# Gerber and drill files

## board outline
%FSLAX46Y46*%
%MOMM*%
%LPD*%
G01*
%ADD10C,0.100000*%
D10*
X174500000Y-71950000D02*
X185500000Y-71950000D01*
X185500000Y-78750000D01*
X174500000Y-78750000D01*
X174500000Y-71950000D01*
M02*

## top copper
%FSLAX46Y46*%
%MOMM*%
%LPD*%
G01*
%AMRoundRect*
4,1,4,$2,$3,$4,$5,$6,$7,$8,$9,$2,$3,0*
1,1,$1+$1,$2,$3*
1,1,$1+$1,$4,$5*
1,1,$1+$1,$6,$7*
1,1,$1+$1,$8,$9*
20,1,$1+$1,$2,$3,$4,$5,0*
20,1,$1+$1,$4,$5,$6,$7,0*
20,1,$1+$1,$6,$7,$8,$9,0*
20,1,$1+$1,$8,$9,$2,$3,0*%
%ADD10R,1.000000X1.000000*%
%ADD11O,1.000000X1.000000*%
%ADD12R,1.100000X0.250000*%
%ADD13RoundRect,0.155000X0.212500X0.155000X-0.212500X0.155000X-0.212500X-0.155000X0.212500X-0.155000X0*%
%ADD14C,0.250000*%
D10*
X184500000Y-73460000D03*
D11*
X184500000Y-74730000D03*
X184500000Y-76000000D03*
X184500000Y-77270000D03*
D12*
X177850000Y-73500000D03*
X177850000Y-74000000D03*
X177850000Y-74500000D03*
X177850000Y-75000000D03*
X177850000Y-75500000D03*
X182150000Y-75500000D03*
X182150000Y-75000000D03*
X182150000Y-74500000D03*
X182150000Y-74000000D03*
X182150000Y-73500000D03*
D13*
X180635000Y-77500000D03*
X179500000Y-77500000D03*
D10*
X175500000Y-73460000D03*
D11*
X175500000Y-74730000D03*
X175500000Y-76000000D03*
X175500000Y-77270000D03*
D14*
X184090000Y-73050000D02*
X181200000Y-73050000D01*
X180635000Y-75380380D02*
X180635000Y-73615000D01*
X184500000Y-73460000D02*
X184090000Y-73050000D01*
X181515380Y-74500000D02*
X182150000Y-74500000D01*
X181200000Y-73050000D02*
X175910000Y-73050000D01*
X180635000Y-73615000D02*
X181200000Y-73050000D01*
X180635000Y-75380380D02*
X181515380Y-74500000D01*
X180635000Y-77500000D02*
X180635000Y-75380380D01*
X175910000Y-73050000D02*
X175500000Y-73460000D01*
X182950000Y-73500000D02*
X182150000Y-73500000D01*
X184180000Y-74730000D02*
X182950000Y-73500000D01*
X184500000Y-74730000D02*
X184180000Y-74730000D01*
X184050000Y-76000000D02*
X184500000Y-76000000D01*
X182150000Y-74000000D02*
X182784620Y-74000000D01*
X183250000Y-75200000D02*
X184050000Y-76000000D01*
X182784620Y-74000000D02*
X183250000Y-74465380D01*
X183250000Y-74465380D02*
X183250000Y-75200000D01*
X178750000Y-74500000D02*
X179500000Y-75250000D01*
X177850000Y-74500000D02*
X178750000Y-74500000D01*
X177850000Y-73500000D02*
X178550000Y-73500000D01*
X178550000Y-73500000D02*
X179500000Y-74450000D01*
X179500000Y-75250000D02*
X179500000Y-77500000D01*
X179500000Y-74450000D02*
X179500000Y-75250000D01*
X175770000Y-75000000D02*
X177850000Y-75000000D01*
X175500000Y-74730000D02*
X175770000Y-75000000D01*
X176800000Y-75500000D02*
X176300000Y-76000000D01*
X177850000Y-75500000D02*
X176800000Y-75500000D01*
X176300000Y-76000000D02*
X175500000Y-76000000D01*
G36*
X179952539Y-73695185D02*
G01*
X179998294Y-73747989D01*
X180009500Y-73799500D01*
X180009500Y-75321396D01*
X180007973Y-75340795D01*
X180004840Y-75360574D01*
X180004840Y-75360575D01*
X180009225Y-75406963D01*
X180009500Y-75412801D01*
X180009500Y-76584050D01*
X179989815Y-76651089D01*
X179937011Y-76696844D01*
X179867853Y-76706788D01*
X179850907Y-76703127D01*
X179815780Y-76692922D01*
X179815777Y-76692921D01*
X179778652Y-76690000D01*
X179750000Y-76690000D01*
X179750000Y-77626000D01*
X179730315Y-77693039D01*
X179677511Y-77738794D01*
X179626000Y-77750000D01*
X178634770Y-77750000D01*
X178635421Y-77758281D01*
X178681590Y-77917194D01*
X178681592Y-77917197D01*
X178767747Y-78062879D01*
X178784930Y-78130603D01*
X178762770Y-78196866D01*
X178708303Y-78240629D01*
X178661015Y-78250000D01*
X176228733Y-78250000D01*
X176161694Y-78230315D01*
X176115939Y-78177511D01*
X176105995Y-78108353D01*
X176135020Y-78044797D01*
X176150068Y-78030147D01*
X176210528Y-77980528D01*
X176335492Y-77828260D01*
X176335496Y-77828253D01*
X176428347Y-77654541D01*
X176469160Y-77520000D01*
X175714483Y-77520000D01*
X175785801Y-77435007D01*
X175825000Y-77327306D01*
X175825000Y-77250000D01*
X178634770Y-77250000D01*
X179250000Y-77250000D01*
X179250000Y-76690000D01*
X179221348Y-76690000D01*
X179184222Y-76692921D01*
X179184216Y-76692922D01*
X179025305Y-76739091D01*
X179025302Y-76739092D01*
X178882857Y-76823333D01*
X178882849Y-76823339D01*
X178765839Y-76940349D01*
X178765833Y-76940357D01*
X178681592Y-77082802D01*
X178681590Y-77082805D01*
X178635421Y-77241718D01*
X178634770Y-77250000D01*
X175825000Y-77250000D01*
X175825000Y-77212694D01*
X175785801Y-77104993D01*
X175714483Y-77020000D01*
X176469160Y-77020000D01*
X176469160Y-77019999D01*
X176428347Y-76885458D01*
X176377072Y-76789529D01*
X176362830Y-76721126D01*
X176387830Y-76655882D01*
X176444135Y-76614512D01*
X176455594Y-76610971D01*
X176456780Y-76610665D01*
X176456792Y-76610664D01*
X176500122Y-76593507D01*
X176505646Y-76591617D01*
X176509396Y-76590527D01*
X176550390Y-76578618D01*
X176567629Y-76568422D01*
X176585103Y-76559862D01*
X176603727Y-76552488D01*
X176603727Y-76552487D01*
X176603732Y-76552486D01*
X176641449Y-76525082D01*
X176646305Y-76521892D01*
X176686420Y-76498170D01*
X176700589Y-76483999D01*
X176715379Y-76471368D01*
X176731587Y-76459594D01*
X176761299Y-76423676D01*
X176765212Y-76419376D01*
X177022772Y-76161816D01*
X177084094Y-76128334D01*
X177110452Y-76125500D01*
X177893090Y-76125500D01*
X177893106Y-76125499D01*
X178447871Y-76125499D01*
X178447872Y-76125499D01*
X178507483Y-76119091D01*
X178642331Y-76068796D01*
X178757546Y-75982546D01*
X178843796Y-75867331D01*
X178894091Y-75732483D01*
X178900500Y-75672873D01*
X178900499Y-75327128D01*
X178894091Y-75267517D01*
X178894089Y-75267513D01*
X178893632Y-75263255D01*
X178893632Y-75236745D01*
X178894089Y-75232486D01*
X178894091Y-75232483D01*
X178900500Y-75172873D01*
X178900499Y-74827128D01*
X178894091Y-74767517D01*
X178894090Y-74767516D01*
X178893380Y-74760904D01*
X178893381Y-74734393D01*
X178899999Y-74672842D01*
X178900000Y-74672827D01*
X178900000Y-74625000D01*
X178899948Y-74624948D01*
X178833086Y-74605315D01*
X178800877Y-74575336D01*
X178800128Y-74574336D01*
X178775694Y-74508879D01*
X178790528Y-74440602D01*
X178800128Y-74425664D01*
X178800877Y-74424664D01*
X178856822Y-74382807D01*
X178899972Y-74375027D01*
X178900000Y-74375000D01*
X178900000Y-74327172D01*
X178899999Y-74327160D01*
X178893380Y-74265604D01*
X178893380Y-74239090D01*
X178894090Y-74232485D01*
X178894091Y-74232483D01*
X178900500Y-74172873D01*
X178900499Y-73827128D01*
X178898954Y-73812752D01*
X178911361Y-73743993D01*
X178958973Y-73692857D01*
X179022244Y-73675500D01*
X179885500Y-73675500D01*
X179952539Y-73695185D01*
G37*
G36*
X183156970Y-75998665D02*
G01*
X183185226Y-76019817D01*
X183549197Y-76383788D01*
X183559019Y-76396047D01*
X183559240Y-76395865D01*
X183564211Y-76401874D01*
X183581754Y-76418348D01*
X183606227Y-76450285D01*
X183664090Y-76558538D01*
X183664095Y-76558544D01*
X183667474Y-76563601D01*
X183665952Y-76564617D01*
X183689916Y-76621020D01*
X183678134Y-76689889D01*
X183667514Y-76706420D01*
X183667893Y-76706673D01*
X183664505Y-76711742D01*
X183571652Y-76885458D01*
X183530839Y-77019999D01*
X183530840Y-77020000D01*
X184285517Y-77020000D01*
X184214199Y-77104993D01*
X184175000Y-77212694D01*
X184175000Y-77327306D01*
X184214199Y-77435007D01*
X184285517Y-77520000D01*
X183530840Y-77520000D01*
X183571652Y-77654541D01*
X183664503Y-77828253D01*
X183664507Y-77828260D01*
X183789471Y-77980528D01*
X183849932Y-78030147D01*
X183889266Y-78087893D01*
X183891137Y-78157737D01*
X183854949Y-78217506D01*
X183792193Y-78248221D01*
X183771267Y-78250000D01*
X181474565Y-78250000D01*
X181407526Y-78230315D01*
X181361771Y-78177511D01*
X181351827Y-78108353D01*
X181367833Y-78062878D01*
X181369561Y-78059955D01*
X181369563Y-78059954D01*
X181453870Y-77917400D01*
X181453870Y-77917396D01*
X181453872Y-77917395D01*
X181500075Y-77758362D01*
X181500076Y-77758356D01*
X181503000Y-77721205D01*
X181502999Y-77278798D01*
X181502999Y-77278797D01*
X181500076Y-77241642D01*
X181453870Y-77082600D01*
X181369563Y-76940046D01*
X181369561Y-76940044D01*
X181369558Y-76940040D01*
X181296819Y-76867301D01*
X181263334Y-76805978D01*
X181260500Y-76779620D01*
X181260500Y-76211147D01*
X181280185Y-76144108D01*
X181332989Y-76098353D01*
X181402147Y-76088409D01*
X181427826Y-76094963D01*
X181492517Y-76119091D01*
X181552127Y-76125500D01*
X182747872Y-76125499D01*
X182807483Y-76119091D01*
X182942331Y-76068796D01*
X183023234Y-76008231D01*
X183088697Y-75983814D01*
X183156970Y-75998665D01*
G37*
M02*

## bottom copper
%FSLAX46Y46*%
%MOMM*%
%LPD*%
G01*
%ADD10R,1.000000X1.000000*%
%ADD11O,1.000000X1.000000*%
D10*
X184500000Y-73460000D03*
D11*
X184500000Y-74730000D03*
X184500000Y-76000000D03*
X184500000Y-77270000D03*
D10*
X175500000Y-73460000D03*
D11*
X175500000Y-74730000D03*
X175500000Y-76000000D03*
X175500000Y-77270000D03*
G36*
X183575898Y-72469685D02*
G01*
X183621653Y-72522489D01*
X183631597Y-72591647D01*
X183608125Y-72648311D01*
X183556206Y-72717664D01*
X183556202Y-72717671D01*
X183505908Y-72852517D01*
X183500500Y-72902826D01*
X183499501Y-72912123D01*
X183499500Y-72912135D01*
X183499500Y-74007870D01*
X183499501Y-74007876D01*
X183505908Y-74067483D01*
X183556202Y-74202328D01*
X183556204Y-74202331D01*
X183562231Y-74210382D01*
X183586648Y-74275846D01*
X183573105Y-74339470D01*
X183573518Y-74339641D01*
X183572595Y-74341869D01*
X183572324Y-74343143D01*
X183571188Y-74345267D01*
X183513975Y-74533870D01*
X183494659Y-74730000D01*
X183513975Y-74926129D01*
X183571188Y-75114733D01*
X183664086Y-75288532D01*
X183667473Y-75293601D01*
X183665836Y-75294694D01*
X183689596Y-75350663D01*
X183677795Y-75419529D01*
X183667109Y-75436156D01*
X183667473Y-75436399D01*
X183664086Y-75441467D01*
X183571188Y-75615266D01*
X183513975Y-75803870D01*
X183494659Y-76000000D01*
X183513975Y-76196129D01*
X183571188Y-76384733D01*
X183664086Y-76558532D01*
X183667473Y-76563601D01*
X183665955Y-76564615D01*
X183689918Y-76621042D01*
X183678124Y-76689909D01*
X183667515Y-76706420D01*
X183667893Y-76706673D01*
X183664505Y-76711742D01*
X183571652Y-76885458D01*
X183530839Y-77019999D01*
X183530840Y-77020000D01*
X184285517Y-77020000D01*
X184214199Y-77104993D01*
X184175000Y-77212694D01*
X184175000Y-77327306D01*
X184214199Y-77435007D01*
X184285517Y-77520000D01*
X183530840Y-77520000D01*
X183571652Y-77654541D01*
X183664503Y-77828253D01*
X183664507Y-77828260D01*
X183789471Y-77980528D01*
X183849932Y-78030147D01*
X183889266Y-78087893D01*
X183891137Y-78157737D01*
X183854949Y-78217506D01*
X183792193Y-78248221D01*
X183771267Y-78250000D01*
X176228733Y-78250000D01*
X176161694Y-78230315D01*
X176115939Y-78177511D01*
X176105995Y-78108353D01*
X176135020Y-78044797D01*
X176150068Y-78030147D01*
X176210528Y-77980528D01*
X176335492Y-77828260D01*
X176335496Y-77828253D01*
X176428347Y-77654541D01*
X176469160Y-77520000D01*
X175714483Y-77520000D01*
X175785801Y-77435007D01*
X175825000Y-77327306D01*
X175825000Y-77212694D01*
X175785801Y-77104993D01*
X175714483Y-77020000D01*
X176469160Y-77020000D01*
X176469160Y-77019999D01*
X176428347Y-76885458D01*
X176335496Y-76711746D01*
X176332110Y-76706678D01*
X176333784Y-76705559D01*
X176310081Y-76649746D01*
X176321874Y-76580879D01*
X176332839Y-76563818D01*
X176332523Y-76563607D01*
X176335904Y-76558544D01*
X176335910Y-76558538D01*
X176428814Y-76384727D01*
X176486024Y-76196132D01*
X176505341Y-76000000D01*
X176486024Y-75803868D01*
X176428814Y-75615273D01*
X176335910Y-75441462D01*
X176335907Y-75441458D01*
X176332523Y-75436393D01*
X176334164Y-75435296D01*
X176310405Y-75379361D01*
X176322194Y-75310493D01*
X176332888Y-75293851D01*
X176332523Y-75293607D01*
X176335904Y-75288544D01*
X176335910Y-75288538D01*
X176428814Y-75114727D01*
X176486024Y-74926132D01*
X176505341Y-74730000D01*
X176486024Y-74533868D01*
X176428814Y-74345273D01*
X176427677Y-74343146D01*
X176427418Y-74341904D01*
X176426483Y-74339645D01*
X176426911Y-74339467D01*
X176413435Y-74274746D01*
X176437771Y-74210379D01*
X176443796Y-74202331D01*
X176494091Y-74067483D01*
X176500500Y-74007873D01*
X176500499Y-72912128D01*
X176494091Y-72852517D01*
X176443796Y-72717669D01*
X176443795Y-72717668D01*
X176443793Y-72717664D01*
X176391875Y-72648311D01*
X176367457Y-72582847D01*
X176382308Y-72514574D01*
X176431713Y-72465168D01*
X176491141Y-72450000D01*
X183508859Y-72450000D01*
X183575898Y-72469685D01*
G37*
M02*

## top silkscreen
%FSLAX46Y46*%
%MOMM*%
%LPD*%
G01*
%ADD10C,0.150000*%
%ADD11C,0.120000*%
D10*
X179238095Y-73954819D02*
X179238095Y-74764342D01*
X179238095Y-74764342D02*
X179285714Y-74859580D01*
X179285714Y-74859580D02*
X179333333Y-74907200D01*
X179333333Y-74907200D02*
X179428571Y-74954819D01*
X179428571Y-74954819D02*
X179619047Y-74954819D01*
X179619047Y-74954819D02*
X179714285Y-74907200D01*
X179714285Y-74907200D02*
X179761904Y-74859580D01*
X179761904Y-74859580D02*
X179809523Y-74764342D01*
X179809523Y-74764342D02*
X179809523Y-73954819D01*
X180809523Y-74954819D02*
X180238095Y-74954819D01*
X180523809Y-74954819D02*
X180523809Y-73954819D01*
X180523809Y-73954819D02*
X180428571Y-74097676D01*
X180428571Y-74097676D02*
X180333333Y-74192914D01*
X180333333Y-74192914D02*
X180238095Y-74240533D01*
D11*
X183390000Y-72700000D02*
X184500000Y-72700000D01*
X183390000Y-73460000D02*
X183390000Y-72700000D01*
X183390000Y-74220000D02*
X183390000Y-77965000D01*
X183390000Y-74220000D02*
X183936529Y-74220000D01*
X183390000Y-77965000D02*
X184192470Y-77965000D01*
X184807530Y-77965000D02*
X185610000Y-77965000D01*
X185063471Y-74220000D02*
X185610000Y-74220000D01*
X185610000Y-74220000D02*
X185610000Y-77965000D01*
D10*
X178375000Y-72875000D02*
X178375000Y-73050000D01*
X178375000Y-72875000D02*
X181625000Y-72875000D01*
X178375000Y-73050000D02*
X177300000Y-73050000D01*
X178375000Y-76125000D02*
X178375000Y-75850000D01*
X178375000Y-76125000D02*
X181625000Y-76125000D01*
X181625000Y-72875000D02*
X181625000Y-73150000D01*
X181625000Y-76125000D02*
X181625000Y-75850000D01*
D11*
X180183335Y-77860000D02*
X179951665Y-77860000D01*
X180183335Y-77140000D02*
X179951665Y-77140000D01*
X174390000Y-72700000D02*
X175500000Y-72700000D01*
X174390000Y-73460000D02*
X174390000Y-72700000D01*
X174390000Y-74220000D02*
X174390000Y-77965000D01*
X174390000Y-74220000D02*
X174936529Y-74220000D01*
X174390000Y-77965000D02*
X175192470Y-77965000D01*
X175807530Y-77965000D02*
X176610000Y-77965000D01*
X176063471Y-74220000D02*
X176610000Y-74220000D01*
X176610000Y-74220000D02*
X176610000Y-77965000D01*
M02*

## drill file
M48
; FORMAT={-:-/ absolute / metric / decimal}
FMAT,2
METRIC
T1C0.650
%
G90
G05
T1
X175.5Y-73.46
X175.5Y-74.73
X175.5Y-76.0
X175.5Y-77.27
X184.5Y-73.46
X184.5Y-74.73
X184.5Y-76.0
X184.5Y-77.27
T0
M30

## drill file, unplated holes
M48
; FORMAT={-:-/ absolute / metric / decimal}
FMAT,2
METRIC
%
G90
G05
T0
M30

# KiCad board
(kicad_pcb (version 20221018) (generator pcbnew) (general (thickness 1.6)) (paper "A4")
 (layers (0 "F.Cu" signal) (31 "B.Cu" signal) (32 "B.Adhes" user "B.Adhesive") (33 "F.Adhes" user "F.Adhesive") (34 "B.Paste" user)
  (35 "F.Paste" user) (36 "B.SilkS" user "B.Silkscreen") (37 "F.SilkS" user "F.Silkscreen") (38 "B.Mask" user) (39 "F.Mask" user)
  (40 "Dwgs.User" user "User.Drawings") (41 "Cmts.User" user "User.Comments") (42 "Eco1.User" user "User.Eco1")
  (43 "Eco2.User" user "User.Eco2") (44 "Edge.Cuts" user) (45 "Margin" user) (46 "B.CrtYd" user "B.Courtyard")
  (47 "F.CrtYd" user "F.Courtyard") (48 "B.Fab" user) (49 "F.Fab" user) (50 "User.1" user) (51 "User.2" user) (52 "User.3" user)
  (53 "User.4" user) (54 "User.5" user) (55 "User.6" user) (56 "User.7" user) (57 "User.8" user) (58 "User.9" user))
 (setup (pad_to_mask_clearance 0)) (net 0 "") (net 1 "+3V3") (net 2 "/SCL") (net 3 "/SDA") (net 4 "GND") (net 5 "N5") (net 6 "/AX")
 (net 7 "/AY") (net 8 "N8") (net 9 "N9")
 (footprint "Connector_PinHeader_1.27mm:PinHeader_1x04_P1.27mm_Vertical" (layer "F.Cu") (at 184.5 73.46)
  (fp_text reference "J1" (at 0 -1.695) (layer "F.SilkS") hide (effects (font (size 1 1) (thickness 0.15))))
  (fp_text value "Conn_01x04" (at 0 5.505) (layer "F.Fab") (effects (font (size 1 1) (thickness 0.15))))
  (fp_line (start -1.11 -0.76) (end 0 -0.76) (stroke (width 0.12) (type solid)) (layer "F.SilkS"))
  (fp_line (start -1.11 0) (end -1.11 -0.76) (stroke (width 0.12) (type solid)) (layer "F.SilkS"))
  (fp_line (start -1.11 0.76) (end -1.11 4.505) (stroke (width 0.12) (type solid)) (layer "F.SilkS"))
  (fp_line (start -1.11 0.76) (end -0.563471 0.76) (stroke (width 0.12) (type solid)) (layer "F.SilkS"))
  (fp_line (start -1.11 4.505) (end -0.30753 4.505) (stroke (width 0.12) (type solid)) (layer "F.SilkS"))
  (fp_line (start 0.30753 4.505) (end 1.11 4.505) (stroke (width 0.12) (type solid)) (layer "F.SilkS"))
  (fp_line (start 0.563471 0.76) (end 1.11 0.76) (stroke (width 0.12) (type solid)) (layer "F.SilkS"))
  (fp_line (start 1.11 0.76) (end 1.11 4.505) (stroke (width 0.12) (type solid)) (layer "F.SilkS"))
  (pad "1" thru_hole rect (at 0 0) (size 1 1) (drill 0.65) (layers "*.Cu" "*.Mask") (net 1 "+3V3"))
  (pad "2" thru_hole oval (at 0 1.27) (size 1 1) (drill 0.65) (layers "*.Cu" "*.Mask") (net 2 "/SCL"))
  (pad "3" thru_hole oval (at 0 2.54) (size 1 1) (drill 0.65) (layers "*.Cu" "*.Mask") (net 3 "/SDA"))
  (pad "4" thru_hole oval (at 0 3.81) (size 1 1) (drill 0.65) (layers "*.Cu" "*.Mask") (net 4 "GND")))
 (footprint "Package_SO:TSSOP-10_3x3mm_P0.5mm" (layer "F.Cu") (at 180 74.5)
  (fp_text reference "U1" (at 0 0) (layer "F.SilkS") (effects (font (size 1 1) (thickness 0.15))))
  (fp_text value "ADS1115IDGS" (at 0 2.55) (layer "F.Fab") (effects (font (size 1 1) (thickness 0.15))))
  (fp_line (start -1.625 -1.625) (end -1.625 -1.45) (stroke (width 0.15) (type solid)) (layer "F.SilkS"))
  (fp_line (start -1.625 -1.625) (end 1.625 -1.625) (stroke (width 0.15) (type solid)) (layer "F.SilkS"))
  (fp_line (start -1.625 -1.45) (end -2.7 -1.45) (stroke (width 0.15) (type solid)) (layer "F.SilkS"))
  (fp_line (start -1.625 1.625) (end -1.625 1.35) (stroke (width 0.15) (type solid)) (layer "F.SilkS"))
  (fp_line (start -1.625 1.625) (end 1.625 1.625) (stroke (width 0.15) (type solid)) (layer "F.SilkS"))
  (fp_line (start 1.625 -1.625) (end 1.625 -1.35) (stroke (width 0.15) (type solid)) (layer "F.SilkS"))
  (fp_line (start 1.625 1.625) (end 1.625 1.35) (stroke (width 0.15) (type solid)) (layer "F.SilkS"))
  (pad "1" smd rect (at -2.15 -1) (size 1.1 0.25) (layers "F.Cu" "F.Paste" "F.Mask") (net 4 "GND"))
  (pad "2" smd rect (at -2.15 -0.5) (size 1.1 0.25) (layers "F.Cu" "F.Paste" "F.Mask") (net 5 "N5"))
  (pad "3" smd rect (at -2.15 0) (size 1.1 0.25) (layers "F.Cu" "F.Paste" "F.Mask") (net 4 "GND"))
  (pad "4" smd rect (at -2.15 0.5) (size 1.1 0.25) (layers "F.Cu" "F.Paste" "F.Mask") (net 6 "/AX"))
  (pad "5" smd rect (at -2.15 1) (size 1.1 0.25) (layers "F.Cu" "F.Paste" "F.Mask") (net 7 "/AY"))
  (pad "6" smd rect (at 2.15 1) (size 1.1 0.25) (layers "F.Cu" "F.Paste" "F.Mask") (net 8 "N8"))
  (pad "7" smd rect (at 2.15 0.5) (size 1.1 0.25) (layers "F.Cu" "F.Paste" "F.Mask") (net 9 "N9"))
  (pad "8" smd rect (at 2.15 0) (size 1.1 0.25) (layers "F.Cu" "F.Paste" "F.Mask") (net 1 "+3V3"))
  (pad "9" smd rect (at 2.15 -0.5) (size 1.1 0.25) (layers "F.Cu" "F.Paste" "F.Mask") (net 3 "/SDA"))
  (pad "10" smd rect (at 2.15 -1) (size 1.1 0.25) (layers "F.Cu" "F.Paste" "F.Mask") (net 2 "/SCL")))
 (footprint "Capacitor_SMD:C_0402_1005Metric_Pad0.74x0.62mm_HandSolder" (layer "F.Cu") (at 180.0675 77.5 180)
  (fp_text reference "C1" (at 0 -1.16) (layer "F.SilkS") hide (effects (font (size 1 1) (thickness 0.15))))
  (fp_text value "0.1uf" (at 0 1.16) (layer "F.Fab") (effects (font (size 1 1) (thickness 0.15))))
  (fp_line (start -0.115835 -0.36) (end 0.115835 -0.36) (stroke (width 0.12) (type solid)) (layer "F.SilkS"))
  (fp_line (start -0.115835 0.36) (end 0.115835 0.36) (stroke (width 0.12) (type solid)) (layer "F.SilkS"))
  (pad "1" smd roundrect (at -0.5675 0 180) (size 0.735 0.62) (layers "F.Cu" "F.Paste" "F.Mask") (roundrect_rratio 0.25) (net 1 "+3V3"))
  (pad "2" smd roundrect (at 0.5675 0 180) (size 0.735 0.62) (layers "F.Cu" "F.Paste" "F.Mask") (roundrect_rratio 0.25) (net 4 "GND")))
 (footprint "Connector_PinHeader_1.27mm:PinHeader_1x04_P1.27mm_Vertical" (layer "F.Cu") (at 175.5 73.46)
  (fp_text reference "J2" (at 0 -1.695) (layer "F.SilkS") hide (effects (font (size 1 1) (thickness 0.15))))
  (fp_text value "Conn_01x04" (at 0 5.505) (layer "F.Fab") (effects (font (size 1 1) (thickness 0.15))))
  (fp_line (start -1.11 -0.76) (end 0 -0.76) (stroke (width 0.12) (type solid)) (layer "F.SilkS"))
  (fp_line (start -1.11 0) (end -1.11 -0.76) (stroke (width 0.12) (type solid)) (layer "F.SilkS"))
  (fp_line (start -1.11 0.76) (end -1.11 4.505) (stroke (width 0.12) (type solid)) (layer "F.SilkS"))
  (fp_line (start -1.11 0.76) (end -0.563471 0.76) (stroke (width 0.12) (type solid)) (layer "F.SilkS"))
  (fp_line (start -1.11 4.505) (end -0.30753 4.505) (stroke (width 0.12) (type solid)) (layer "F.SilkS"))
  (fp_line (start 0.30753 4.505) (end 1.11 4.505) (stroke (width 0.12) (type solid)) (layer "F.SilkS"))
  (fp_line (start 0.563471 0.76) (end 1.11 0.76) (stroke (width 0.12) (type solid)) (layer "F.SilkS"))
  (fp_line (start 1.11 0.76) (end 1.11 4.505) (stroke (width 0.12) (type solid)) (layer "F.SilkS"))
  (pad "1" thru_hole rect (at 0 0) (size 1 1) (drill 0.65) (layers "*.Cu" "*.Mask") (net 1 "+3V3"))
  (pad "2" thru_hole oval (at 0 1.27) (size 1 1) (drill 0.65) (layers "*.Cu" "*.Mask") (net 6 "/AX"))
  (pad "3" thru_hole oval (at 0 2.54) (size 1 1) (drill 0.65) (layers "*.Cu" "*.Mask") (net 7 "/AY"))
  (pad "4" thru_hole oval (at 0 3.81) (size 1 1) (drill 0.65) (layers "*.Cu" "*.Mask") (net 4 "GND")))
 (gr_rect (start 174.5 71.95) (end 185.5 78.75) (stroke (width 0.1) (type default)) (fill none) (layer "Edge.Cuts"))
 (segment (start 184.09 73.05) (end 181.2 73.05) (width 0.25) (layer "F.Cu") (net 1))
 (segment (start 180.635 75.38038) (end 180.635 73.615) (width 0.25) (layer "F.Cu") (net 1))
 (segment (start 184.5 73.46) (end 184.09 73.05) (width 0.25) (layer "F.Cu") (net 1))
 (segment (start 181.51538 74.5) (end 182.15 74.5) (width 0.25) (layer "F.Cu") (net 1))
 (segment (start 181.2 73.05) (end 175.91 73.05) (width 0.25) (layer "F.Cu") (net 1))
 (segment (start 180.635 73.615) (end 181.2 73.05) (width 0.25) (layer "F.Cu") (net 1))
 (segment (start 180.635 75.38038) (end 181.51538 74.5) (width 0.25) (layer "F.Cu") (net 1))
 (segment (start 180.635 77.5) (end 180.635 75.38038) (width 0.25) (layer "F.Cu") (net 1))
 (segment (start 175.91 73.05) (end 175.5 73.46) (width 0.25) (layer "F.Cu") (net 1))
 (segment (start 182.95 73.5) (end 182.15 73.5) (width 0.25) (layer "F.Cu") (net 2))
 (segment (start 184.18 74.73) (end 182.95 73.5) (width 0.25) (layer "F.Cu") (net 2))
 (segment (start 184.5 74.73) (end 184.18 74.73) (width 0.25) (layer "F.Cu") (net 2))
 (segment (start 184.05 76) (end 184.5 76) (width 0.25) (layer "F.Cu") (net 3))
 (segment (start 182.15 74) (end 182.78462 74) (width 0.25) (layer "F.Cu") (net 3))
 (segment (start 183.25 75.2) (end 184.05 76) (width 0.25) (layer "F.Cu") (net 3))
 (segment (start 182.78462 74) (end 183.25 74.46538) (width 0.25) (layer "F.Cu") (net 3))
 (segment (start 183.25 74.46538) (end 183.25 75.2) (width 0.25) (layer "F.Cu") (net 3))
 (segment (start 178.75 74.5) (end 179.5 75.25) (width 0.25) (layer "F.Cu") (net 4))
 (segment (start 177.85 74.5) (end 178.75 74.5) (width 0.25) (layer "F.Cu") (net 4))
 (segment (start 177.85 73.5) (end 178.55 73.5) (width 0.25) (layer "F.Cu") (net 4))
 (segment (start 178.55 73.5) (end 179.5 74.45) (width 0.25) (layer "F.Cu") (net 4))
 (segment (start 179.5 75.25) (end 179.5 77.5) (width 0.25) (layer "F.Cu") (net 4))
 (segment (start 179.5 74.45) (end 179.5 75.25) (width 0.25) (layer "F.Cu") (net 4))
 (segment (start 175.77 75) (end 177.85 75) (width 0.25) (layer "F.Cu") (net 6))
 (segment (start 175.5 74.73) (end 175.77 75) (width 0.25) (layer "F.Cu") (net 6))
 (segment (start 176.8 75.5) (end 176.3 76) (width 0.25) (layer "F.Cu") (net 7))
 (segment (start 177.85 75.5) (end 176.8 75.5) (width 0.25) (layer "F.Cu") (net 7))
 (segment (start 176.3 76) (end 175.5 76) (width 0.25) (layer "F.Cu") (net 7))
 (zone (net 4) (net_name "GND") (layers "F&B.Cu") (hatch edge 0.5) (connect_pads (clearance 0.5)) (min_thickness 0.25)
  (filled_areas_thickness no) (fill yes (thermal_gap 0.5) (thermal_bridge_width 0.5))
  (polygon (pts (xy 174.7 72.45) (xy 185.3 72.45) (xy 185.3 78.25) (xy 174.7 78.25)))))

